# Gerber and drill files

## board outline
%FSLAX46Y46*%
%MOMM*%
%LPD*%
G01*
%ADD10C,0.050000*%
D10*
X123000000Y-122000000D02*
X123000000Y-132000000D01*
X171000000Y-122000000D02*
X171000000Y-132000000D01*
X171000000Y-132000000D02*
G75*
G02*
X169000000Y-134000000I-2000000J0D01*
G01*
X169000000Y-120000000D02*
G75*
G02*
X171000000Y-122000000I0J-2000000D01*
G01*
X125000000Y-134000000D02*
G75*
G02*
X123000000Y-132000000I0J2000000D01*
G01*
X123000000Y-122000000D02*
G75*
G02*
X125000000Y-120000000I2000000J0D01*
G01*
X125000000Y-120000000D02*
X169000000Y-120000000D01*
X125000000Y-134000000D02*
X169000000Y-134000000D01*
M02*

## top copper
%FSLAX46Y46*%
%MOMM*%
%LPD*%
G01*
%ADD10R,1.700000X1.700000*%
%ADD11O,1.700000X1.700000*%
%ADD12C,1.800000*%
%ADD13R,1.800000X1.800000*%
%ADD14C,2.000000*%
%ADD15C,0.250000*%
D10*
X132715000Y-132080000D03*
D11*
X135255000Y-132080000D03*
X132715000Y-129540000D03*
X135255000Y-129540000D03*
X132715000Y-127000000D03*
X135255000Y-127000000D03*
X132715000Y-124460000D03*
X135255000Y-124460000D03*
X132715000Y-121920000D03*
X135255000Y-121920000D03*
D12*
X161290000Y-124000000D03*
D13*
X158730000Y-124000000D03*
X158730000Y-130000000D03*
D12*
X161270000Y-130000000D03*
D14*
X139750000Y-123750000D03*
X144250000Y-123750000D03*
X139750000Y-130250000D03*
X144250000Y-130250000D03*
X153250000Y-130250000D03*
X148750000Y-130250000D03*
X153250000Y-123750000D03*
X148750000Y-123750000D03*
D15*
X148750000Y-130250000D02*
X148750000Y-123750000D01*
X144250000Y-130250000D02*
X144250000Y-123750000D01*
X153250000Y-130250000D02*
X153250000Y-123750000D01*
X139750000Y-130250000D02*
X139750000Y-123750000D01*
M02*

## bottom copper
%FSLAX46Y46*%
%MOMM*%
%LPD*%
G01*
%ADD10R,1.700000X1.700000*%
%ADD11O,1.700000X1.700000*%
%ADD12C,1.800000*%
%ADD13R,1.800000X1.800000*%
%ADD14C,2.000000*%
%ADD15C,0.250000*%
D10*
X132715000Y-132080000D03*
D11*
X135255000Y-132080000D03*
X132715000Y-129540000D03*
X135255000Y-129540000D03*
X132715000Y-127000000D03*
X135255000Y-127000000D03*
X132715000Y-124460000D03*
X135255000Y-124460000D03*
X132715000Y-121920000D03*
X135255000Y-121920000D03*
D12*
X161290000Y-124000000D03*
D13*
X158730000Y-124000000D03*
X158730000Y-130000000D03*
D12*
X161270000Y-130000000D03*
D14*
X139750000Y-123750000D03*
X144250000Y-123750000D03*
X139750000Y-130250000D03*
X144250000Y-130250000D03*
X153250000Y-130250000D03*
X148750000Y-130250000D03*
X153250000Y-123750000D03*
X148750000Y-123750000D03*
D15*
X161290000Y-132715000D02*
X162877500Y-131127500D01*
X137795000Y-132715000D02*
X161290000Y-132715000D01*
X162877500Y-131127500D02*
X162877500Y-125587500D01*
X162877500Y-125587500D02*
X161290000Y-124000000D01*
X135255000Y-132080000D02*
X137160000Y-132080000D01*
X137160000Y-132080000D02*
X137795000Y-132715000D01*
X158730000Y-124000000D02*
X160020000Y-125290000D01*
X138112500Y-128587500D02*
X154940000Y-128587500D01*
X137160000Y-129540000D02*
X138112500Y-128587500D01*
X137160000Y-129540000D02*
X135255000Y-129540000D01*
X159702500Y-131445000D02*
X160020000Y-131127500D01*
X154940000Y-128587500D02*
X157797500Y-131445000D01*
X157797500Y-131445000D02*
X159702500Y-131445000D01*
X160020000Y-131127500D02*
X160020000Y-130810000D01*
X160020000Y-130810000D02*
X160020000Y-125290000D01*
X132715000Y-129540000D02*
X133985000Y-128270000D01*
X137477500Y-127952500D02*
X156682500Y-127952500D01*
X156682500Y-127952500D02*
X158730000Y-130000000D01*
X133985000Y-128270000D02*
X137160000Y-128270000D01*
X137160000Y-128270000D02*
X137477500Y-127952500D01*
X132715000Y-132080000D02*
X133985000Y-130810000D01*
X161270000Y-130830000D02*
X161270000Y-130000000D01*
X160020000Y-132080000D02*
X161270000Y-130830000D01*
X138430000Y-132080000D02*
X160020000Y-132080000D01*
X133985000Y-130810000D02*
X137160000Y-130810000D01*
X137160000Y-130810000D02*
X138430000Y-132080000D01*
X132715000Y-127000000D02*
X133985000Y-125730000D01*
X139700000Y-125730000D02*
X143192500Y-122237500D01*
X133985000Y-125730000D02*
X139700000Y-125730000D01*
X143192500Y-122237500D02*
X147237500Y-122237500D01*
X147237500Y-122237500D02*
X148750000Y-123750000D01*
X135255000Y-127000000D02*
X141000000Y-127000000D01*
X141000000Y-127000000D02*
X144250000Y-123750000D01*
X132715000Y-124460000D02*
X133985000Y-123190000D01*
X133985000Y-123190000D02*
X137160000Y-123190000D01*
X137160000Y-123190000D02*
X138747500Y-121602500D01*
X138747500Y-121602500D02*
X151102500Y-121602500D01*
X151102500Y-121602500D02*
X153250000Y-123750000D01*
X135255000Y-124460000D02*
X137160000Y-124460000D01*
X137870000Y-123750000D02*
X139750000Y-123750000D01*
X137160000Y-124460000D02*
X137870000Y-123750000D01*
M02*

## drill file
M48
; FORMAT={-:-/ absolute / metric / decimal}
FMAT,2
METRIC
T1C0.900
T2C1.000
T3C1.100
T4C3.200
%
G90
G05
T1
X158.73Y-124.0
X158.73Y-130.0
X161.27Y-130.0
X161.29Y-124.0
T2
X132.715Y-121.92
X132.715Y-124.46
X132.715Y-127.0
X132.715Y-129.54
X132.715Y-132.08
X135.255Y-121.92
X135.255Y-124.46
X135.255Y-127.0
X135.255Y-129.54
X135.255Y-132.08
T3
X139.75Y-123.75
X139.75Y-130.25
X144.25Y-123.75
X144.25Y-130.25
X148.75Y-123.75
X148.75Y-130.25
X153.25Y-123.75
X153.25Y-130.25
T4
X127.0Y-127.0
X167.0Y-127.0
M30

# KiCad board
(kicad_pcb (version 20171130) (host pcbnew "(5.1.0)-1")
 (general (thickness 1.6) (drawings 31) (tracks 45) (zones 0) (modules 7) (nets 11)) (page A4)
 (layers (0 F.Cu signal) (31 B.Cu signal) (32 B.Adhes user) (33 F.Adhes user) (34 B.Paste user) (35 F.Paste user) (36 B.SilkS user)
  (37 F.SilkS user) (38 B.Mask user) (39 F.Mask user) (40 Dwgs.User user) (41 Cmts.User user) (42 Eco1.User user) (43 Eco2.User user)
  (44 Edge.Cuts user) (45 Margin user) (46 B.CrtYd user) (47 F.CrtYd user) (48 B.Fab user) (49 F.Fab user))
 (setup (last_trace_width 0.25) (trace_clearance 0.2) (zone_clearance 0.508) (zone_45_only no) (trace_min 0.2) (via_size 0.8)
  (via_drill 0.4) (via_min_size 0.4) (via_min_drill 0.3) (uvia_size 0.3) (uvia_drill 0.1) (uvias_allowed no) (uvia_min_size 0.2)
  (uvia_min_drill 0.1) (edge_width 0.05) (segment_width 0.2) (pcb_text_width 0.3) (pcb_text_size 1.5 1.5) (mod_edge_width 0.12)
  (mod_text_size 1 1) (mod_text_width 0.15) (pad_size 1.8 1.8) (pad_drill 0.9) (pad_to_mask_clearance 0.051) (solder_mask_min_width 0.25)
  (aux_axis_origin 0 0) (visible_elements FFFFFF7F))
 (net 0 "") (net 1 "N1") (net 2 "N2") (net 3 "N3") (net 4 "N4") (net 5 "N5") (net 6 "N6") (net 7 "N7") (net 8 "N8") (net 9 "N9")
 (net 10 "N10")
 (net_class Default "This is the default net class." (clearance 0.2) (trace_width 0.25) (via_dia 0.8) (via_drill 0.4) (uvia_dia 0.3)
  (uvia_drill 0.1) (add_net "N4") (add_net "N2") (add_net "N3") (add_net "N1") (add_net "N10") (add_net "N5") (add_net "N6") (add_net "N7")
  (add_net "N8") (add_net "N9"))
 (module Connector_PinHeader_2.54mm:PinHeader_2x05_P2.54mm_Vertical (layer B.Cu) (at 132.715 132.08)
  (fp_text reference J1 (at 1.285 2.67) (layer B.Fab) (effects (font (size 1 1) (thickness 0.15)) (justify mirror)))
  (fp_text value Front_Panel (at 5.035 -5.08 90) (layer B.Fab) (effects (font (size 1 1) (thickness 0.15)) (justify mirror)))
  (pad 1 thru_hole rect (at 0 0) (size 1.7 1.7) (drill 1) (layers *.Cu *.Mask) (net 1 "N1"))
  (pad 2 thru_hole oval (at 2.54 0) (size 1.7 1.7) (drill 1) (layers *.Cu *.Mask) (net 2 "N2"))
  (pad 3 thru_hole oval (at 0 -2.54) (size 1.7 1.7) (drill 1) (layers *.Cu *.Mask) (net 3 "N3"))
  (pad 4 thru_hole oval (at 2.54 -2.54) (size 1.7 1.7) (drill 1) (layers *.Cu *.Mask) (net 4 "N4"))
  (pad 5 thru_hole oval (at 0 -5.08) (size 1.7 1.7) (drill 1) (layers *.Cu *.Mask) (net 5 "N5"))
  (pad 6 thru_hole oval (at 2.54 -5.08) (size 1.7 1.7) (drill 1) (layers *.Cu *.Mask) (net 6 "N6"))
  (pad 7 thru_hole oval (at 0 -7.62) (size 1.7 1.7) (drill 1) (layers *.Cu *.Mask) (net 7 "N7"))
  (pad 8 thru_hole oval (at 2.54 -7.62) (size 1.7 1.7) (drill 1) (layers *.Cu *.Mask) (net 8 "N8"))
  (pad 9 thru_hole oval (at 0 -10.16) (size 1.7 1.7) (drill 1) (layers *.Cu *.Mask) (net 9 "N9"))
  (pad 10 thru_hole oval (at 2.54 -10.16) (size 1.7 1.7) (drill 1) (layers *.Cu *.Mask) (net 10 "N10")))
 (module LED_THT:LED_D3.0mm (layer F.Cu) (at 158.75 124)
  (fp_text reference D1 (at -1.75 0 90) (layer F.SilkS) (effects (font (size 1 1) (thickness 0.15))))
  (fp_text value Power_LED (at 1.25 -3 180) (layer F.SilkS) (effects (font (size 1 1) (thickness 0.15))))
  (pad 2 thru_hole circle (at 2.54 0) (size 1.8 1.8) (drill 0.9) (layers *.Cu *.Mask) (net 2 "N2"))
  (pad 1 thru_hole rect (at -0.02 0) (size 1.8 1.8) (drill 0.9) (layers *.Cu *.Mask) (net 4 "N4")))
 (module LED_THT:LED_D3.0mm (layer F.Cu) (at 158.73 130)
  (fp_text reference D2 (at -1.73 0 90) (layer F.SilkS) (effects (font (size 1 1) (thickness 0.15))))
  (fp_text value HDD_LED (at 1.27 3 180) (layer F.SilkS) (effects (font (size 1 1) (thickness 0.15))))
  (pad 1 thru_hole rect (at 0 0) (size 1.8 1.8) (drill 0.9) (layers *.Cu *.Mask) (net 3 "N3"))
  (pad 2 thru_hole circle (at 2.54 0) (size 1.8 1.8) (drill 0.9) (layers *.Cu *.Mask) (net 1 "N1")))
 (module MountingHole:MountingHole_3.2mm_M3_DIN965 (layer F.Cu) (at 127 127)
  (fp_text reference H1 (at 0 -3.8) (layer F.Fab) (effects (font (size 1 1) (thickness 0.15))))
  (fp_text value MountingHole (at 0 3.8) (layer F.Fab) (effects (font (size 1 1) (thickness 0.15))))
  (pad 1 np_thru_hole circle (at 0 0) (size 3.2 3.2) (drill 3.2) (layers *.Cu *.Mask)))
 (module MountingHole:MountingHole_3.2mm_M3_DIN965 (layer F.Cu) (at 167 127)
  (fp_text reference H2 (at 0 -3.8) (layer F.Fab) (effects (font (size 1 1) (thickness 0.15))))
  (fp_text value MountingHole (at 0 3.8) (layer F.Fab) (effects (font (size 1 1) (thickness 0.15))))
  (pad 1 np_thru_hole circle (at 0 0) (size 3.2 3.2) (drill 3.2) (layers *.Cu *.Mask)))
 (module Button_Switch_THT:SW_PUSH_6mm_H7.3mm (layer F.Cu) (at 139.75 130.25 90)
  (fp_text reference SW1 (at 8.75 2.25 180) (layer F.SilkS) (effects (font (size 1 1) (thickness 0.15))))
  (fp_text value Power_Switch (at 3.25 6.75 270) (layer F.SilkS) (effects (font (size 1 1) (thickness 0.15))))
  (pad 1 thru_hole circle (at 6.5 0 180) (size 2 2) (drill 1.1) (layers *.Cu *.Mask) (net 8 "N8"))
  (pad 2 thru_hole circle (at 6.5 4.5 180) (size 2 2) (drill 1.1) (layers *.Cu *.Mask) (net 6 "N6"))
  (pad 1 thru_hole circle (at 0 0 180) (size 2 2) (drill 1.1) (layers *.Cu *.Mask) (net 8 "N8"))
  (pad 2 thru_hole circle (at 0 4.5 180) (size 2 2) (drill 1.1) (layers *.Cu *.Mask) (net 6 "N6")))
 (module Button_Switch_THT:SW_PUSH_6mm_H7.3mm (layer F.Cu) (at 148.75 130.25 90)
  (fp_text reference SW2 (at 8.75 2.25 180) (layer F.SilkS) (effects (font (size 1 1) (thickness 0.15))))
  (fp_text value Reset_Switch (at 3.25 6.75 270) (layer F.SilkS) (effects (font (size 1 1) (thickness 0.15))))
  (pad 2 thru_hole circle (at 0 4.5 180) (size 2 2) (drill 1.1) (layers *.Cu *.Mask) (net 7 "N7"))
  (pad 1 thru_hole circle (at 0 0 180) (size 2 2) (drill 1.1) (layers *.Cu *.Mask) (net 5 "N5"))
  (pad 2 thru_hole circle (at 6.5 4.5 180) (size 2 2) (drill 1.1) (layers *.Cu *.Mask) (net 7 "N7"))
  (pad 1 thru_hole circle (at 6.5 0 180) (size 2 2) (drill 1.1) (layers *.Cu *.Mask) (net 5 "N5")))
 (gr_line (start 123 122) (end 123 132) (angle 90) (layer Edge.Cuts) (width 0.05))
 (gr_line (start 171 122) (end 171 132) (angle 90) (layer Edge.Cuts) (width 0.05))
 (gr_arc (start 169 132) (end 171 132) (angle 90) (layer Edge.Cuts) (width 0.05))
 (gr_arc (start 169 122) (end 169 120) (angle 90) (layer Edge.Cuts) (width 0.05))
 (gr_arc (start 125 132) (end 125 134) (angle 90) (layer Edge.Cuts) (width 0.05))
 (gr_arc (start 125 122) (end 123 122) (angle 90) (layer Edge.Cuts) (width 0.05))
 (gr_line (start 125 120) (end 169 120) (angle 90) (layer Edge.Cuts) (width 0.05))
 (gr_line (start 125 134) (end 169 134) (angle 90) (layer Edge.Cuts) (width 0.05))
 (segment (start 161.29 132.715) (end 162.8775 131.1275) (width 0.25) (layer B.Cu) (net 2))
 (segment (start 137.795 132.715) (end 161.29 132.715) (width 0.25) (layer B.Cu) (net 2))
 (segment (start 162.8775 131.1275) (end 162.8775 125.5875) (width 0.25) (layer B.Cu) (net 2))
 (segment (start 162.8775 125.5875) (end 161.29 124) (width 0.25) (layer B.Cu) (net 2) (status 800000))
 (segment (start 135.255 132.08) (end 137.16 132.08) (width 0.25) (layer B.Cu) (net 2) (status 400000))
 (segment (start 137.16 132.08) (end 137.795 132.715) (width 0.25) (layer B.Cu) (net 2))
 (segment (start 158.73 124) (end 160.02 125.29) (width 0.25) (layer B.Cu) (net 4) (status 400000))
 (segment (start 138.1125 128.5875) (end 154.94 128.5875) (width 0.25) (layer B.Cu) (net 4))
 (segment (start 137.16 129.54) (end 138.1125 128.5875) (width 0.25) (layer B.Cu) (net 4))
 (segment (start 137.16 129.54) (end 135.255 129.54) (width 0.25) (layer B.Cu) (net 4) (status 800000))
 (segment (start 159.7025 131.445) (end 160.02 131.1275) (width 0.25) (layer B.Cu) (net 4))
 (segment (start 154.94 128.5875) (end 157.7975 131.445) (width 0.25) (layer B.Cu) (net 4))
 (segment (start 157.7975 131.445) (end 159.7025 131.445) (width 0.25) (layer B.Cu) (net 4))
 (segment (start 160.02 131.1275) (end 160.02 130.81) (width 0.25) (layer B.Cu) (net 4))
 (segment (start 160.02 130.81) (end 160.02 125.29) (width 0.25) (layer B.Cu) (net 4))
 (segment (start 132.715 129.54) (end 133.985 128.27) (width 0.25) (layer B.Cu) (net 3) (status 400000))
 (segment (start 137.4775 127.9525) (end 156.6825 127.9525) (width 0.25) (layer B.Cu) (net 3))
 (segment (start 156.6825 127.9525) (end 158.73 130) (width 0.25) (layer B.Cu) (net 3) (status 800000))
 (segment (start 133.985 128.27) (end 137.16 128.27) (width 0.25) (layer B.Cu) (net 3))
 (segment (start 137.16 128.27) (end 137.4775 127.9525) (width 0.25) (layer B.Cu) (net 3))
 (segment (start 132.715 132.08) (end 133.985 130.81) (width 0.25) (layer B.Cu) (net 1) (status 400000))
 (segment (start 161.27 130.83) (end 161.27 130) (width 0.25) (layer B.Cu) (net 1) (status C00000))
 (segment (start 160.02 132.08) (end 161.27 130.83) (width 0.25) (layer B.Cu) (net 1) (status 800000))
 (segment (start 138.43 132.08) (end 160.02 132.08) (width 0.25) (layer B.Cu) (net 1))
 (segment (start 133.985 130.81) (end 137.16 130.81) (width 0.25) (layer B.Cu) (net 1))
 (segment (start 137.16 130.81) (end 138.43 132.08) (width 0.25) (layer B.Cu) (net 1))
 (segment (start 148.75 130.25) (end 148.75 123.75) (width 0.25) (layer F.Cu) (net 5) (status C00000))
 (segment (start 132.715 127) (end 133.985 125.73) (width 0.25) (layer B.Cu) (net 5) (status 400000))
 (segment (start 139.7 125.73) (end 143.1925 122.2375) (width 0.25) (layer B.Cu) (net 5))
 (segment (start 133.985 125.73) (end 139.7 125.73) (width 0.25) (layer B.Cu) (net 5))
 (segment (start 143.1925 122.2375) (end 147.2375 122.2375) (width 0.25) (layer B.Cu) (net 5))
 (segment (start 147.2375 122.2375) (end 148.75 123.75) (width 0.25) (layer B.Cu) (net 5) (status 800000))
 (segment (start 144.25 130.25) (end 144.25 123.75) (width 0.25) (layer F.Cu) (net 6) (status C00000))
 (segment (start 135.255 127) (end 141 127) (width 0.25) (layer B.Cu) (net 6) (status 400000))
 (segment (start 141 127) (end 144.25 123.75) (width 0.25) (layer B.Cu) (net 6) (status 800000))
 (segment (start 153.25 130.25) (end 153.25 123.75) (width 0.25) (layer F.Cu) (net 7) (status C00000))
 (segment (start 132.715 124.46) (end 133.985 123.19) (width 0.25) (layer B.Cu) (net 7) (status 400000))
 (segment (start 133.985 123.19) (end 137.16 123.19) (width 0.25) (layer B.Cu) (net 7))
 (segment (start 137.16 123.19) (end 138.7475 121.6025) (width 0.25) (layer B.Cu) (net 7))
 (segment (start 138.7475 121.6025) (end 151.1025 121.6025) (width 0.25) (layer B.Cu) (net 7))
 (segment (start 151.1025 121.6025) (end 153.25 123.75) (width 0.25) (layer B.Cu) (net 7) (status 800000))
 (segment (start 139.75 130.25) (end 139.75 123.75) (width 0.25) (layer F.Cu) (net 8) (status C00000))
 (segment (start 135.255 124.46) (end 137.16 124.46) (width 0.25) (layer B.Cu) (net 8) (status 400000))
 (segment (start 137.87 123.75) (end 139.75 123.75) (width 0.25) (layer B.Cu) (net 8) (status 800000))
 (segment (start 137.16 124.46) (end 137.87 123.75) (width 0.25) (layer B.Cu) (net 8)))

